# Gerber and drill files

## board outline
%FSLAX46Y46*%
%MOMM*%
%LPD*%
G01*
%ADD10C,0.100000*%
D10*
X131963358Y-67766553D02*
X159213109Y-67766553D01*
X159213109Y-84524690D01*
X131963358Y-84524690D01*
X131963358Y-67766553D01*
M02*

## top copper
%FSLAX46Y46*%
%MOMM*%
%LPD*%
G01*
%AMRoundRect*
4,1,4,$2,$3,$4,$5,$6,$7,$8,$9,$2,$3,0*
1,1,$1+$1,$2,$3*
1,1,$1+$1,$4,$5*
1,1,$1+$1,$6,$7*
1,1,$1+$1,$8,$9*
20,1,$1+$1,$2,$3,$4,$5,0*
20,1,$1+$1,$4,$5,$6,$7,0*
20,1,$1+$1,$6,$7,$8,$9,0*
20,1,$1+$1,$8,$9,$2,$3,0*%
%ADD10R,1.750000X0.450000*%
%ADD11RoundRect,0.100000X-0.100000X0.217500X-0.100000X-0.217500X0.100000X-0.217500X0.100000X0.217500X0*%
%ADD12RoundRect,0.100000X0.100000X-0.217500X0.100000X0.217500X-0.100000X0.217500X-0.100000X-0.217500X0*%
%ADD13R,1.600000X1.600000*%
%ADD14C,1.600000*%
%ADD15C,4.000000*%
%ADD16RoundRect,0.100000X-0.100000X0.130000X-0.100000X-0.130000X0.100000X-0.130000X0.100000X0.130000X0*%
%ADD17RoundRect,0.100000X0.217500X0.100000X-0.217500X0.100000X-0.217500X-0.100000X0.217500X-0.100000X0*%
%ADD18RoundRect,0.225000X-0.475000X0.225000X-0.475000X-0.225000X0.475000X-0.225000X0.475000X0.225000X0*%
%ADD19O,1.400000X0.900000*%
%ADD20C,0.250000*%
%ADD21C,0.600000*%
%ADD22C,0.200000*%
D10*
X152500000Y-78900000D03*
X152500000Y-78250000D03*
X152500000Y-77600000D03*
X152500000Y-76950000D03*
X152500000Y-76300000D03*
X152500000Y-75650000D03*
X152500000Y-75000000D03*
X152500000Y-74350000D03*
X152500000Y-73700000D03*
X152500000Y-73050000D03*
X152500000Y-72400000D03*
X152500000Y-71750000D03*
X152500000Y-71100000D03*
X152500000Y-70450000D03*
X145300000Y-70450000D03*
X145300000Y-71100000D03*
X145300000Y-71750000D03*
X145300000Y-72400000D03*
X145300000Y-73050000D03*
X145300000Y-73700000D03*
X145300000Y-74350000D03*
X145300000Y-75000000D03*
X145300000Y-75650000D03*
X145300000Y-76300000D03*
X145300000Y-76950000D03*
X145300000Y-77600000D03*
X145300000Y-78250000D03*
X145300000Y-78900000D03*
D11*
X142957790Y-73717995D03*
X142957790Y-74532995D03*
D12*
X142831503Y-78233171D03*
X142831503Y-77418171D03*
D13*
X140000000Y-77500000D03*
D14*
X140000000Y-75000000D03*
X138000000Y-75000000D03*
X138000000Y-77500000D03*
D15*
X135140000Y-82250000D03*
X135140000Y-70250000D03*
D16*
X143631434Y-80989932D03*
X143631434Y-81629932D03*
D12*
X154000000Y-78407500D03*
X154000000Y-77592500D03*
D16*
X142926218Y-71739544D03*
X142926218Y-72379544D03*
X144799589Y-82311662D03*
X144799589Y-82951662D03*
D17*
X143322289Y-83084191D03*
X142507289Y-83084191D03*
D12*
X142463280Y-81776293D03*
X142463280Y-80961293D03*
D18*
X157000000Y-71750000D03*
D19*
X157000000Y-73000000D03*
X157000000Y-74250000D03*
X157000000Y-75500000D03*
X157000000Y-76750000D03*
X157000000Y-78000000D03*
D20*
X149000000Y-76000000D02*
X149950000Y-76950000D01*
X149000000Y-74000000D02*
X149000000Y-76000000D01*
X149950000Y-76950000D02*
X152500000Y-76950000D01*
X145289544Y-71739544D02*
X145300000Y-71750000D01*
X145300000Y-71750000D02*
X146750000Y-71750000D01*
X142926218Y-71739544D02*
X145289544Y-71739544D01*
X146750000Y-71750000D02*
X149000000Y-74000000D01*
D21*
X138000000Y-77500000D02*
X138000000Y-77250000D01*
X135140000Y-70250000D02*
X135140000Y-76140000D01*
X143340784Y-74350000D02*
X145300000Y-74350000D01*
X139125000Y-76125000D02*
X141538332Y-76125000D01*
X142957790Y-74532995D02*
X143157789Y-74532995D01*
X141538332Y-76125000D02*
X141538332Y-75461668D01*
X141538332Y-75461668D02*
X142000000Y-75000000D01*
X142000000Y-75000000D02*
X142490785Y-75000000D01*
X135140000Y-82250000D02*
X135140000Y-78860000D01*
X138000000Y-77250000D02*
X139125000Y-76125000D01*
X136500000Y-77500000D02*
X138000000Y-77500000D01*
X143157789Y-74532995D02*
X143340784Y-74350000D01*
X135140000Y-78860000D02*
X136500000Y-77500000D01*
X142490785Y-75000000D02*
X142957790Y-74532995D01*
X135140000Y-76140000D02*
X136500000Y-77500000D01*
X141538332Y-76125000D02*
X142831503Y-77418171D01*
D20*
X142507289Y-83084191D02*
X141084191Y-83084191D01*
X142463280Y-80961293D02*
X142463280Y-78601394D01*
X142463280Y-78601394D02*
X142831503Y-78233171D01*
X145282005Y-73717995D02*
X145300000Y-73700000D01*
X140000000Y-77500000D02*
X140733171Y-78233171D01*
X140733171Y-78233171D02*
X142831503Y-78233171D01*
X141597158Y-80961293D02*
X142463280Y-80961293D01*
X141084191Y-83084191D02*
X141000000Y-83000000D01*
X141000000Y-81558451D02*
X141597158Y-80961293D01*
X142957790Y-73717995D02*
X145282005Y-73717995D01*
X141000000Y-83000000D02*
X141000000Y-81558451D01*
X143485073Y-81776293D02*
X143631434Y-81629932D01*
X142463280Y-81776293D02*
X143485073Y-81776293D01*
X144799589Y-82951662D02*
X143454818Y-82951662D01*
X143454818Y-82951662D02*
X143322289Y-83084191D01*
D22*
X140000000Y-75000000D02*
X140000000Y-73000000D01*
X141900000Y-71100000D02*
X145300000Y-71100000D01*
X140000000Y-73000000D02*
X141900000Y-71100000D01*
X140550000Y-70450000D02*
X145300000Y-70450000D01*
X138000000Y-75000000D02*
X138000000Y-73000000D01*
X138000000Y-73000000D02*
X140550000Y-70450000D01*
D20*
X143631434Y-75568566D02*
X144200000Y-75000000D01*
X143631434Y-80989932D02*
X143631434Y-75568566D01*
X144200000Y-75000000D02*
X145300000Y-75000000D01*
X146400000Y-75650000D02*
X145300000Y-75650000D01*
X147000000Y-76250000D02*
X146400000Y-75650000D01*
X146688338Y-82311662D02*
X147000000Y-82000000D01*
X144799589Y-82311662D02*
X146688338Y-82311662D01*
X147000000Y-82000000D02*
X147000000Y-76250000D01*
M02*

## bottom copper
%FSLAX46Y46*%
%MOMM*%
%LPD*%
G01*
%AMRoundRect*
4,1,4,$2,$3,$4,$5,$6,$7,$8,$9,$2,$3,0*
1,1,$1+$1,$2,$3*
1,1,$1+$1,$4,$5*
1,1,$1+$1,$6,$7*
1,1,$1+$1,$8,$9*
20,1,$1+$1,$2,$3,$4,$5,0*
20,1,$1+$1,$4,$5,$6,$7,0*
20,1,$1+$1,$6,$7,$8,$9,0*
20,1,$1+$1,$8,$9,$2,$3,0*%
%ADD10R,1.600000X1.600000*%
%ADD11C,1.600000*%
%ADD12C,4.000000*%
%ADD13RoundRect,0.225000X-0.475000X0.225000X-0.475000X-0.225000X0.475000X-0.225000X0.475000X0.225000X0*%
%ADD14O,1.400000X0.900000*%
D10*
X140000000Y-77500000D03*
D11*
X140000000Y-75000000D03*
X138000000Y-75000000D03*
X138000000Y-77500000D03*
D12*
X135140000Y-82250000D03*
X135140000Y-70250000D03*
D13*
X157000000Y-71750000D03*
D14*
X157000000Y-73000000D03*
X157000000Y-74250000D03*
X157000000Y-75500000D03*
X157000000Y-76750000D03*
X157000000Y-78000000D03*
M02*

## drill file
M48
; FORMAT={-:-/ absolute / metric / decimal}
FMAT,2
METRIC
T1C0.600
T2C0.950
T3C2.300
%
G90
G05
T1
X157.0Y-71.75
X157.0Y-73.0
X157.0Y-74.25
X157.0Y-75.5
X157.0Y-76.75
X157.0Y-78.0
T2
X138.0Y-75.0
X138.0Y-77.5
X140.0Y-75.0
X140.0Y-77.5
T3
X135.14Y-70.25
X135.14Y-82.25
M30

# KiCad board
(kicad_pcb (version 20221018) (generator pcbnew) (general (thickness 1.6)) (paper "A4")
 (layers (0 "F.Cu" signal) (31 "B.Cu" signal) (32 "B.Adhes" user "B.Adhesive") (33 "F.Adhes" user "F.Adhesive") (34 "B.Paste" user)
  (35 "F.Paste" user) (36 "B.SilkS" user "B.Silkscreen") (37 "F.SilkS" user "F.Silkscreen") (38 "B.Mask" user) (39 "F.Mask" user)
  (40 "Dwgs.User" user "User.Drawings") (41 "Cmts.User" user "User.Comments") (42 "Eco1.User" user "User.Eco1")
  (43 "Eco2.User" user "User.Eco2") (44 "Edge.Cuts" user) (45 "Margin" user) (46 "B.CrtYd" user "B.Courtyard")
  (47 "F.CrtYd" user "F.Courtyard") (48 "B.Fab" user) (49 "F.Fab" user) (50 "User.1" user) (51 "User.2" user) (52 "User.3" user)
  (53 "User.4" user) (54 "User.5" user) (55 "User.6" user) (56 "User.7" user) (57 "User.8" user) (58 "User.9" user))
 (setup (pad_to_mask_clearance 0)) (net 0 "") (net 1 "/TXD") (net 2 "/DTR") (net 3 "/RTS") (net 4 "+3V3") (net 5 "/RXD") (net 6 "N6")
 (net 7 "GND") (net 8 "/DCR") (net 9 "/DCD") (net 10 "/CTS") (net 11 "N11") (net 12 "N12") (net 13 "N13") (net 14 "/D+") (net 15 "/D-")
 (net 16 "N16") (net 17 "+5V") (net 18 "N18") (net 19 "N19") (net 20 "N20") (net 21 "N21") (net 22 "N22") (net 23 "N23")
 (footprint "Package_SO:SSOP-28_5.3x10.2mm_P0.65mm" (layer "F.Cu") (at 148.9 74.675 180)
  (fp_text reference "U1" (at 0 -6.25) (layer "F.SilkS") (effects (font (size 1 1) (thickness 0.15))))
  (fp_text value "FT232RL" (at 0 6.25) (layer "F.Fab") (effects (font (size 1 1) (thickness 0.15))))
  (pad "1" smd rect (at -3.6 -4.225 180) (size 1.75 0.45) (layers "F.Cu" "F.Paste" "F.Mask") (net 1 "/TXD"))
  (pad "2" smd rect (at -3.6 -3.575 180) (size 1.75 0.45) (layers "F.Cu" "F.Paste" "F.Mask") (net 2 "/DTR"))
  (pad "3" smd rect (at -3.6 -2.925 180) (size 1.75 0.45) (layers "F.Cu" "F.Paste" "F.Mask") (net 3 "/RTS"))
  (pad "4" smd rect (at -3.6 -2.275 180) (size 1.75 0.45) (layers "F.Cu" "F.Paste" "F.Mask") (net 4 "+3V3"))
  (pad "5" smd rect (at -3.6 -1.625 180) (size 1.75 0.45) (layers "F.Cu" "F.Paste" "F.Mask") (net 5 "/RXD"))
  (pad "6" smd rect (at -3.6 -0.975 180) (size 1.75 0.45) (layers "F.Cu" "F.Paste" "F.Mask") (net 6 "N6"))
  (pad "7" smd rect (at -3.6 -0.325 180) (size 1.75 0.45) (layers "F.Cu" "F.Paste" "F.Mask") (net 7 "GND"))
  (pad "8" smd rect (at -3.6 0.325 180) (size 1.75 0.45) (layers "F.Cu" "F.Paste" "F.Mask"))
  (pad "9" smd rect (at -3.6 0.975 180) (size 1.75 0.45) (layers "F.Cu" "F.Paste" "F.Mask") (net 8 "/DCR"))
  (pad "10" smd rect (at -3.6 1.625 180) (size 1.75 0.45) (layers "F.Cu" "F.Paste" "F.Mask") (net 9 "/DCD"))
  (pad "11" smd rect (at -3.6 2.275 180) (size 1.75 0.45) (layers "F.Cu" "F.Paste" "F.Mask") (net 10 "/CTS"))
  (pad "12" smd rect (at -3.6 2.925 180) (size 1.75 0.45) (layers "F.Cu" "F.Paste" "F.Mask") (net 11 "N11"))
  (pad "13" smd rect (at -3.6 3.575 180) (size 1.75 0.45) (layers "F.Cu" "F.Paste" "F.Mask") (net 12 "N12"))
  (pad "14" smd rect (at -3.6 4.225 180) (size 1.75 0.45) (layers "F.Cu" "F.Paste" "F.Mask") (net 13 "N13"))
  (pad "15" smd rect (at 3.6 4.225 180) (size 1.75 0.45) (layers "F.Cu" "F.Paste" "F.Mask") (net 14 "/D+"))
  (pad "16" smd rect (at 3.6 3.575 180) (size 1.75 0.45) (layers "F.Cu" "F.Paste" "F.Mask") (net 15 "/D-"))
  (pad "17" smd rect (at 3.6 2.925 180) (size 1.75 0.45) (layers "F.Cu" "F.Paste" "F.Mask") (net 4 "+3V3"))
  (pad "18" smd rect (at 3.6 2.275 180) (size 1.75 0.45) (layers "F.Cu" "F.Paste" "F.Mask") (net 7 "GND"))
  (pad "19" smd rect (at 3.6 1.625 180) (size 1.75 0.45) (layers "F.Cu" "F.Paste" "F.Mask") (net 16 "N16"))
  (pad "20" smd rect (at 3.6 0.975 180) (size 1.75 0.45) (layers "F.Cu" "F.Paste" "F.Mask") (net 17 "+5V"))
  (pad "21" smd rect (at 3.6 0.325 180) (size 1.75 0.45) (layers "F.Cu" "F.Paste" "F.Mask") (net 7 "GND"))
  (pad "22" smd rect (at 3.6 -0.325 180) (size 1.75 0.45) (layers "F.Cu" "F.Paste" "F.Mask") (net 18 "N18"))
  (pad "23" smd rect (at 3.6 -0.975 180) (size 1.75 0.45) (layers "F.Cu" "F.Paste" "F.Mask") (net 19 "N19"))
  (pad "24" smd rect (at 3.6 -1.625 180) (size 1.75 0.45) (layers "F.Cu" "F.Paste" "F.Mask"))
  (pad "25" smd rect (at 3.6 -2.275 180) (size 1.75 0.45) (layers "F.Cu" "F.Paste" "F.Mask") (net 7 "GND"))
  (pad "26" smd rect (at 3.6 -2.925 180) (size 1.75 0.45) (layers "F.Cu" "F.Paste" "F.Mask") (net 7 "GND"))
  (pad "27" smd rect (at 3.6 -3.575 180) (size 1.75 0.45) (layers "F.Cu" "F.Paste" "F.Mask") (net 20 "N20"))
  (pad "28" smd rect (at 3.6 -4.225 180) (size 1.75 0.45) (layers "F.Cu" "F.Paste" "F.Mask") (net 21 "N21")))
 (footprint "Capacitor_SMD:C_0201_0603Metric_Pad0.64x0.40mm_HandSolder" (layer "F.Cu") (at 142.95779 74.125495 -90)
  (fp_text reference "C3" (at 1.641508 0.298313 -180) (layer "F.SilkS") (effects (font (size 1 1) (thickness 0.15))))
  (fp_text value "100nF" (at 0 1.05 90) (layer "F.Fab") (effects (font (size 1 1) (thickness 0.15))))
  (pad "" smd roundrect (at -0.4325 0 270) (size 0.458 0.36) (layers "F.Paste") (roundrect_rratio 0.25))
  (pad "" smd roundrect (at 0.4325 0 270) (size 0.458 0.36) (layers "F.Paste") (roundrect_rratio 0.25))
  (pad "1" smd roundrect (at -0.4075 0 270) (size 0.635 0.4) (layers "F.Cu" "F.Mask") (roundrect_rratio 0.25) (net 17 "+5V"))
  (pad "2" smd roundrect (at 0.4075 0 270) (size 0.635 0.4) (layers "F.Cu" "F.Mask") (roundrect_rratio 0.25) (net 7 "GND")))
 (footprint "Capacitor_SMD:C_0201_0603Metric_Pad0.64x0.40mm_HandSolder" (layer "F.Cu") (at 142.831503 77.825671 90)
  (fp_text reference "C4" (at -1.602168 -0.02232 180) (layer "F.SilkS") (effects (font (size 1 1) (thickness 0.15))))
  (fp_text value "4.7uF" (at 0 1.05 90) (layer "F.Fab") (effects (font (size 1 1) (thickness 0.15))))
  (pad "" smd roundrect (at -0.4325 0 90) (size 0.458 0.36) (layers "F.Paste") (roundrect_rratio 0.25))
  (pad "" smd roundrect (at 0.4325 0 90) (size 0.458 0.36) (layers "F.Paste") (roundrect_rratio 0.25))
  (pad "1" smd roundrect (at -0.4075 0 90) (size 0.635 0.4) (layers "F.Cu" "F.Mask") (roundrect_rratio 0.25) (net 17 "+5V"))
  (pad "2" smd roundrect (at 0.4075 0 90) (size 0.635 0.4) (layers "F.Cu" "F.Mask") (roundrect_rratio 0.25) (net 7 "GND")))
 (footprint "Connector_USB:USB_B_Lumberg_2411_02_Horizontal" (layer "F.Cu") (at 140 77.5 180)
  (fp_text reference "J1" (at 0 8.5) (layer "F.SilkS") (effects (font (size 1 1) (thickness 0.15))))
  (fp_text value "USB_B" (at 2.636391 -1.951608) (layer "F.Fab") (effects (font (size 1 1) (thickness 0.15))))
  (pad "1" thru_hole rect (at 0 0 270) (size 1.6 1.6) (drill 0.95) (layers "*.Cu" "*.Mask") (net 17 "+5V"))
  (pad "2" thru_hole circle (at 0 2.5 270) (size 1.6 1.6) (drill 0.95) (layers "*.Cu" "*.Mask") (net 15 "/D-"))
  (pad "3" thru_hole circle (at 2 2.5 270) (size 1.6 1.6) (drill 0.95) (layers "*.Cu" "*.Mask") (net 14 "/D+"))
  (pad "4" thru_hole circle (at 2 0 270) (size 1.6 1.6) (drill 0.95) (layers "*.Cu" "*.Mask") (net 7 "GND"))
  (pad "5" thru_hole circle (at 4.86 -4.75 270) (size 4 4) (drill 2.3) (layers "*.Cu" "*.Mask") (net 7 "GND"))
  (pad "5" thru_hole circle (at 4.86 7.25 270) (size 4 4) (drill 2.3) (layers "*.Cu" "*.Mask") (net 7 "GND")))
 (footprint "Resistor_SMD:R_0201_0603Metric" (layer "F.Cu") (at 143.631434 81.309932 -90)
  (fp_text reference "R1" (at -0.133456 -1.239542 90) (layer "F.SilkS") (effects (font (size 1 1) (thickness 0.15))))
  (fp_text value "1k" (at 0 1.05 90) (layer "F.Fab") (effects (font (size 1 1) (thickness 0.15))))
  (pad "" smd roundrect (at -0.345 0 270) (size 0.318 0.36) (layers "F.Paste") (roundrect_rratio 0.25))
  (pad "" smd roundrect (at 0.345 0 270) (size 0.318 0.36) (layers "F.Paste") (roundrect_rratio 0.25))
  (pad "1" smd roundrect (at -0.32 0 270) (size 0.46 0.4) (layers "F.Cu" "F.Mask") (roundrect_rratio 0.25) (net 18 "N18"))
  (pad "2" smd roundrect (at 0.32 0 270) (size 0.46 0.4) (layers "F.Cu" "F.Mask") (roundrect_rratio 0.25) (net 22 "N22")))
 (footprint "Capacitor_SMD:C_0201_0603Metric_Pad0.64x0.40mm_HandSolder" (layer "F.Cu") (at 154 78 90)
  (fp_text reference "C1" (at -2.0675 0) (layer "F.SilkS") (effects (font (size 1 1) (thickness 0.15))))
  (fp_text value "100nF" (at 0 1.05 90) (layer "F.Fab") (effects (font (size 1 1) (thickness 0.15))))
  (pad "" smd roundrect (at -0.4325 0 90) (size 0.458 0.36) (layers "F.Paste") (roundrect_rratio 0.25))
  (pad "" smd roundrect (at 0.4325 0 90) (size 0.458 0.36) (layers "F.Paste") (roundrect_rratio 0.25))
  (pad "1" smd roundrect (at -0.4075 0 90) (size 0.635 0.4) (layers "F.Cu" "F.Mask") (roundrect_rratio 0.25) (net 4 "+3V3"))
  (pad "2" smd roundrect (at 0.4075 0 90) (size 0.635 0.4) (layers "F.Cu" "F.Mask") (roundrect_rratio 0.25) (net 7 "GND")))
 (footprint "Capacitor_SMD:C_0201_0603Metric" (layer "F.Cu") (at 142.926218 72.059544 -90)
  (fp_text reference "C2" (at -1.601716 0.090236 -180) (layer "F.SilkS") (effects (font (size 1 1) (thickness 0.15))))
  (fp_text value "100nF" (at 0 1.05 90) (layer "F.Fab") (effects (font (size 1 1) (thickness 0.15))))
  (pad "" smd roundrect (at -0.345 0 270) (size 0.318 0.36) (layers "F.Paste") (roundrect_rratio 0.25))
  (pad "" smd roundrect (at 0.345 0 270) (size 0.318 0.36) (layers "F.Paste") (roundrect_rratio 0.25))
  (pad "1" smd roundrect (at -0.32 0 270) (size 0.46 0.4) (layers "F.Cu" "F.Mask") (roundrect_rratio 0.25) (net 4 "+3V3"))
  (pad "2" smd roundrect (at 0.32 0 270) (size 0.46 0.4) (layers "F.Cu" "F.Mask") (roundrect_rratio 0.25) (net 7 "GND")))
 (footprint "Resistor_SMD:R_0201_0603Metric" (layer "F.Cu") (at 144.799589 82.631662 -90)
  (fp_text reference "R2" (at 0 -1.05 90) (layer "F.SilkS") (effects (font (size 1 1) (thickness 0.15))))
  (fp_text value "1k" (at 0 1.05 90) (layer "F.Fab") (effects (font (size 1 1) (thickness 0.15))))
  (pad "" smd roundrect (at -0.345 0 270) (size 0.318 0.36) (layers "F.Paste") (roundrect_rratio 0.25))
  (pad "" smd roundrect (at 0.345 0 270) (size 0.318 0.36) (layers "F.Paste") (roundrect_rratio 0.25))
  (pad "1" smd roundrect (at -0.32 0 270) (size 0.46 0.4) (layers "F.Cu" "F.Mask") (roundrect_rratio 0.25) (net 19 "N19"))
  (pad "2" smd roundrect (at 0.32 0 270) (size 0.46 0.4) (layers "F.Cu" "F.Mask") (roundrect_rratio 0.25) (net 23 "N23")))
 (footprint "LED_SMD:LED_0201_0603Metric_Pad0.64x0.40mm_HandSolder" (layer "F.Cu") (at 142.914789 83.084191 180)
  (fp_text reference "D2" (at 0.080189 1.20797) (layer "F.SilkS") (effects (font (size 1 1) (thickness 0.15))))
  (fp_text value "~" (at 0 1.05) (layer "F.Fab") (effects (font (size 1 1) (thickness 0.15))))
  (pad "" smd roundrect (at -0.4325 0 180) (size 0.458 0.36) (layers "F.Paste") (roundrect_rratio 0.25))
  (pad "" smd roundrect (at 0.4325 0 180) (size 0.458 0.36) (layers "F.Paste") (roundrect_rratio 0.25))
  (pad "1" smd roundrect (at -0.4075 0 180) (size 0.635 0.4) (layers "F.Cu" "F.Mask") (roundrect_rratio 0.25) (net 23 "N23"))
  (pad "2" smd roundrect (at 0.4075 0 180) (size 0.635 0.4) (layers "F.Cu" "F.Mask") (roundrect_rratio 0.25) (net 17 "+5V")))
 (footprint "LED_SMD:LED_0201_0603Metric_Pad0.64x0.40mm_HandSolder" (layer "F.Cu") (at 142.46328 81.368793 90)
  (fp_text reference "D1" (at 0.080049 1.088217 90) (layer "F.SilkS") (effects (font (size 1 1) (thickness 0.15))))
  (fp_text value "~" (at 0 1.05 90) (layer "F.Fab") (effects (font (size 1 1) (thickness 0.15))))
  (pad "" smd roundrect (at -0.4325 0 90) (size 0.458 0.36) (layers "F.Paste") (roundrect_rratio 0.25))
  (pad "" smd roundrect (at 0.4325 0 90) (size 0.458 0.36) (layers "F.Paste") (roundrect_rratio 0.25))
  (pad "1" smd roundrect (at -0.4075 0 90) (size 0.635 0.4) (layers "F.Cu" "F.Mask") (roundrect_rratio 0.25) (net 22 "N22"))
  (pad "2" smd roundrect (at 0.4075 0 90) (size 0.635 0.4) (layers "F.Cu" "F.Mask") (roundrect_rratio 0.25) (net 17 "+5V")))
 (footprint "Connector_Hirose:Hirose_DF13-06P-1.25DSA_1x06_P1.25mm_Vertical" (layer "B.Cu") (at 157 71.75 -90)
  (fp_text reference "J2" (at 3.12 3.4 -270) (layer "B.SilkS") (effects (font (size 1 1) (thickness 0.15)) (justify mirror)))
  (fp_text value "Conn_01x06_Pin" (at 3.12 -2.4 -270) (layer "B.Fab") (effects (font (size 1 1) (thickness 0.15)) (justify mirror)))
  (pad "1" thru_hole roundrect (at 0 0 270) (size 0.9 1.4) (drill 0.6) (layers "*.Cu" "*.Mask") (roundrect_rratio 0.25) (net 2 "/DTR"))
  (pad "2" thru_hole oval (at 1.25 0 270) (size 0.9 1.4) (drill 0.6) (layers "*.Cu" "*.Mask") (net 5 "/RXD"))
  (pad "3" thru_hole oval (at 2.5 0 270) (size 0.9 1.4) (drill 0.6) (layers "*.Cu" "*.Mask") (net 1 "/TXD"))
  (pad "4" thru_hole oval (at 3.75 0 270) (size 0.9 1.4) (drill 0.6) (layers "*.Cu" "*.Mask") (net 17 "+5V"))
  (pad "5" thru_hole oval (at 5 0 270) (size 0.9 1.4) (drill 0.6) (layers "*.Cu" "*.Mask") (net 4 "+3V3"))
  (pad "6" thru_hole oval (at 6.25 0 270) (size 0.9 1.4) (drill 0.6) (layers "*.Cu" "*.Mask") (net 7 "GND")))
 (gr_rect (start 131.963358 67.766553) (end 159.213109 84.52469) (stroke (width 0.1) (type default)) (fill none) (layer "Edge.Cuts"))
 (segment (start 149 76) (end 149.95 76.95) (width 0.25) (layer "F.Cu") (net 4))
 (segment (start 149 74) (end 149 76) (width 0.25) (layer "F.Cu") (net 4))
 (segment (start 149.95 76.95) (end 152.5 76.95) (width 0.25) (layer "F.Cu") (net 4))
 (segment (start 145.289544 71.739544) (end 145.3 71.75) (width 0.25) (layer "F.Cu") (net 4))
 (segment (start 145.3 71.75) (end 146.75 71.75) (width 0.25) (layer "F.Cu") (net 4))
 (segment (start 142.926218 71.739544) (end 145.289544 71.739544) (width 0.25) (layer "F.Cu") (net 4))
 (segment (start 146.75 71.75) (end 149 74) (width 0.25) (layer "F.Cu") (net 4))
 (segment (start 138 77.5) (end 138 77.25) (width 0.6) (layer "F.Cu") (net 7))
 (segment (start 135.14 70.25) (end 135.14 76.14) (width 0.6) (layer "F.Cu") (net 7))
 (segment (start 143.340784 74.35) (end 145.3 74.35) (width 0.6) (layer "F.Cu") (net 7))
 (segment (start 139.125 76.125) (end 141.538332 76.125) (width 0.6) (layer "F.Cu") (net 7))
 (segment (start 142.95779 74.532995) (end 143.157789 74.532995) (width 0.6) (layer "F.Cu") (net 7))
 (segment (start 141.538332 76.125) (end 141.538332 75.461668) (width 0.6) (layer "F.Cu") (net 7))
 (segment (start 141.538332 75.461668) (end 142 75) (width 0.6) (layer "F.Cu") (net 7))
 (segment (start 142 75) (end 142.490785 75) (width 0.6) (layer "F.Cu") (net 7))
 (segment (start 135.14 82.25) (end 135.14 78.86) (width 0.6) (layer "F.Cu") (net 7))
 (segment (start 138 77.25) (end 139.125 76.125) (width 0.6) (layer "F.Cu") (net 7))
 (segment (start 136.5 77.5) (end 138 77.5) (width 0.6) (layer "F.Cu") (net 7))
 (segment (start 143.157789 74.532995) (end 143.340784 74.35) (width 0.6) (layer "F.Cu") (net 7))
 (segment (start 135.14 78.86) (end 136.5 77.5) (width 0.6) (layer "F.Cu") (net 7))
 (segment (start 142.490785 75) (end 142.95779 74.532995) (width 0.6) (layer "F.Cu") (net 7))
 (segment (start 135.14 76.14) (end 136.5 77.5) (width 0.6) (layer "F.Cu") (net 7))
 (segment (start 141.538332 76.125) (end 142.831503 77.418171) (width 0.6) (layer "F.Cu") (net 7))
 (segment (start 142.507289 83.084191) (end 141.084191 83.084191) (width 0.25) (layer "F.Cu") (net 17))
 (segment (start 142.46328 80.961293) (end 142.46328 78.601394) (width 0.25) (layer "F.Cu") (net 17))
 (segment (start 142.46328 78.601394) (end 142.831503 78.233171) (width 0.25) (layer "F.Cu") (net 17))
 (segment (start 145.282005 73.717995) (end 145.3 73.7) (width 0.25) (layer "F.Cu") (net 17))
 (segment (start 140 77.5) (end 140.733171 78.233171) (width 0.25) (layer "F.Cu") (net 17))
 (segment (start 140.733171 78.233171) (end 142.831503 78.233171) (width 0.25) (layer "F.Cu") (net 17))
 (segment (start 141.597158 80.961293) (end 142.46328 80.961293) (width 0.25) (layer "F.Cu") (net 17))
 (segment (start 141.084191 83.084191) (end 141 83) (width 0.25) (layer "F.Cu") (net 17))
 (segment (start 141 81.558451) (end 141.597158 80.961293) (width 0.25) (layer "F.Cu") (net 17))
 (segment (start 142.95779 73.717995) (end 145.282005 73.717995) (width 0.25) (layer "F.Cu") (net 17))
 (segment (start 141 83) (end 141 81.558451) (width 0.25) (layer "F.Cu") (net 17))
 (segment (start 143.485073 81.776293) (end 143.631434 81.629932) (width 0.25) (layer "F.Cu") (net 22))
 (segment (start 142.46328 81.776293) (end 143.485073 81.776293) (width 0.25) (layer "F.Cu") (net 22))
 (segment (start 144.799589 82.951662) (end 143.454818 82.951662) (width 0.25) (layer "F.Cu") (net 23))
 (segment (start 143.454818 82.951662) (end 143.322289 83.084191) (width 0.25) (layer "F.Cu") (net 23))
 (segment (start 140 75) (end 140 73) (width 0.2) (layer "F.Cu") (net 15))
 (segment (start 141.9 71.1) (end 145.3 71.1) (width 0.2) (layer "F.Cu") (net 15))
 (segment (start 140 73) (end 141.9 71.1) (width 0.2) (layer "F.Cu") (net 15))
 (segment (start 140.55 70.45) (end 145.3 70.45) (width 0.2) (layer "F.Cu") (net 14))
 (segment (start 138 75) (end 138 73) (width 0.2) (layer "F.Cu") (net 14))
 (segment (start 138 73) (end 140.55 70.45) (width 0.2) (layer "F.Cu") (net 14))
 (segment (start 143.631434 75.568566) (end 144.2 75) (width 0.25) (layer "F.Cu") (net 18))
 (segment (start 143.631434 80.989932) (end 143.631434 75.568566) (width 0.25) (layer "F.Cu") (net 18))
 (segment (start 144.2 75) (end 145.3 75) (width 0.25) (layer "F.Cu") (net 18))
 (segment (start 146.4 75.65) (end 145.3 75.65) (width 0.25) (layer "F.Cu") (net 19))
 (segment (start 147 76.25) (end 146.4 75.65) (width 0.25) (layer "F.Cu") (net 19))
 (segment (start 146.688338 82.311662) (end 147 82) (width 0.25) (layer "F.Cu") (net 19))
 (segment (start 144.799589 82.311662) (end 146.688338 82.311662) (width 0.25) (layer "F.Cu") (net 19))
 (segment (start 147 82) (end 147 76.25) (width 0.25) (layer "F.Cu") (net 19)))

